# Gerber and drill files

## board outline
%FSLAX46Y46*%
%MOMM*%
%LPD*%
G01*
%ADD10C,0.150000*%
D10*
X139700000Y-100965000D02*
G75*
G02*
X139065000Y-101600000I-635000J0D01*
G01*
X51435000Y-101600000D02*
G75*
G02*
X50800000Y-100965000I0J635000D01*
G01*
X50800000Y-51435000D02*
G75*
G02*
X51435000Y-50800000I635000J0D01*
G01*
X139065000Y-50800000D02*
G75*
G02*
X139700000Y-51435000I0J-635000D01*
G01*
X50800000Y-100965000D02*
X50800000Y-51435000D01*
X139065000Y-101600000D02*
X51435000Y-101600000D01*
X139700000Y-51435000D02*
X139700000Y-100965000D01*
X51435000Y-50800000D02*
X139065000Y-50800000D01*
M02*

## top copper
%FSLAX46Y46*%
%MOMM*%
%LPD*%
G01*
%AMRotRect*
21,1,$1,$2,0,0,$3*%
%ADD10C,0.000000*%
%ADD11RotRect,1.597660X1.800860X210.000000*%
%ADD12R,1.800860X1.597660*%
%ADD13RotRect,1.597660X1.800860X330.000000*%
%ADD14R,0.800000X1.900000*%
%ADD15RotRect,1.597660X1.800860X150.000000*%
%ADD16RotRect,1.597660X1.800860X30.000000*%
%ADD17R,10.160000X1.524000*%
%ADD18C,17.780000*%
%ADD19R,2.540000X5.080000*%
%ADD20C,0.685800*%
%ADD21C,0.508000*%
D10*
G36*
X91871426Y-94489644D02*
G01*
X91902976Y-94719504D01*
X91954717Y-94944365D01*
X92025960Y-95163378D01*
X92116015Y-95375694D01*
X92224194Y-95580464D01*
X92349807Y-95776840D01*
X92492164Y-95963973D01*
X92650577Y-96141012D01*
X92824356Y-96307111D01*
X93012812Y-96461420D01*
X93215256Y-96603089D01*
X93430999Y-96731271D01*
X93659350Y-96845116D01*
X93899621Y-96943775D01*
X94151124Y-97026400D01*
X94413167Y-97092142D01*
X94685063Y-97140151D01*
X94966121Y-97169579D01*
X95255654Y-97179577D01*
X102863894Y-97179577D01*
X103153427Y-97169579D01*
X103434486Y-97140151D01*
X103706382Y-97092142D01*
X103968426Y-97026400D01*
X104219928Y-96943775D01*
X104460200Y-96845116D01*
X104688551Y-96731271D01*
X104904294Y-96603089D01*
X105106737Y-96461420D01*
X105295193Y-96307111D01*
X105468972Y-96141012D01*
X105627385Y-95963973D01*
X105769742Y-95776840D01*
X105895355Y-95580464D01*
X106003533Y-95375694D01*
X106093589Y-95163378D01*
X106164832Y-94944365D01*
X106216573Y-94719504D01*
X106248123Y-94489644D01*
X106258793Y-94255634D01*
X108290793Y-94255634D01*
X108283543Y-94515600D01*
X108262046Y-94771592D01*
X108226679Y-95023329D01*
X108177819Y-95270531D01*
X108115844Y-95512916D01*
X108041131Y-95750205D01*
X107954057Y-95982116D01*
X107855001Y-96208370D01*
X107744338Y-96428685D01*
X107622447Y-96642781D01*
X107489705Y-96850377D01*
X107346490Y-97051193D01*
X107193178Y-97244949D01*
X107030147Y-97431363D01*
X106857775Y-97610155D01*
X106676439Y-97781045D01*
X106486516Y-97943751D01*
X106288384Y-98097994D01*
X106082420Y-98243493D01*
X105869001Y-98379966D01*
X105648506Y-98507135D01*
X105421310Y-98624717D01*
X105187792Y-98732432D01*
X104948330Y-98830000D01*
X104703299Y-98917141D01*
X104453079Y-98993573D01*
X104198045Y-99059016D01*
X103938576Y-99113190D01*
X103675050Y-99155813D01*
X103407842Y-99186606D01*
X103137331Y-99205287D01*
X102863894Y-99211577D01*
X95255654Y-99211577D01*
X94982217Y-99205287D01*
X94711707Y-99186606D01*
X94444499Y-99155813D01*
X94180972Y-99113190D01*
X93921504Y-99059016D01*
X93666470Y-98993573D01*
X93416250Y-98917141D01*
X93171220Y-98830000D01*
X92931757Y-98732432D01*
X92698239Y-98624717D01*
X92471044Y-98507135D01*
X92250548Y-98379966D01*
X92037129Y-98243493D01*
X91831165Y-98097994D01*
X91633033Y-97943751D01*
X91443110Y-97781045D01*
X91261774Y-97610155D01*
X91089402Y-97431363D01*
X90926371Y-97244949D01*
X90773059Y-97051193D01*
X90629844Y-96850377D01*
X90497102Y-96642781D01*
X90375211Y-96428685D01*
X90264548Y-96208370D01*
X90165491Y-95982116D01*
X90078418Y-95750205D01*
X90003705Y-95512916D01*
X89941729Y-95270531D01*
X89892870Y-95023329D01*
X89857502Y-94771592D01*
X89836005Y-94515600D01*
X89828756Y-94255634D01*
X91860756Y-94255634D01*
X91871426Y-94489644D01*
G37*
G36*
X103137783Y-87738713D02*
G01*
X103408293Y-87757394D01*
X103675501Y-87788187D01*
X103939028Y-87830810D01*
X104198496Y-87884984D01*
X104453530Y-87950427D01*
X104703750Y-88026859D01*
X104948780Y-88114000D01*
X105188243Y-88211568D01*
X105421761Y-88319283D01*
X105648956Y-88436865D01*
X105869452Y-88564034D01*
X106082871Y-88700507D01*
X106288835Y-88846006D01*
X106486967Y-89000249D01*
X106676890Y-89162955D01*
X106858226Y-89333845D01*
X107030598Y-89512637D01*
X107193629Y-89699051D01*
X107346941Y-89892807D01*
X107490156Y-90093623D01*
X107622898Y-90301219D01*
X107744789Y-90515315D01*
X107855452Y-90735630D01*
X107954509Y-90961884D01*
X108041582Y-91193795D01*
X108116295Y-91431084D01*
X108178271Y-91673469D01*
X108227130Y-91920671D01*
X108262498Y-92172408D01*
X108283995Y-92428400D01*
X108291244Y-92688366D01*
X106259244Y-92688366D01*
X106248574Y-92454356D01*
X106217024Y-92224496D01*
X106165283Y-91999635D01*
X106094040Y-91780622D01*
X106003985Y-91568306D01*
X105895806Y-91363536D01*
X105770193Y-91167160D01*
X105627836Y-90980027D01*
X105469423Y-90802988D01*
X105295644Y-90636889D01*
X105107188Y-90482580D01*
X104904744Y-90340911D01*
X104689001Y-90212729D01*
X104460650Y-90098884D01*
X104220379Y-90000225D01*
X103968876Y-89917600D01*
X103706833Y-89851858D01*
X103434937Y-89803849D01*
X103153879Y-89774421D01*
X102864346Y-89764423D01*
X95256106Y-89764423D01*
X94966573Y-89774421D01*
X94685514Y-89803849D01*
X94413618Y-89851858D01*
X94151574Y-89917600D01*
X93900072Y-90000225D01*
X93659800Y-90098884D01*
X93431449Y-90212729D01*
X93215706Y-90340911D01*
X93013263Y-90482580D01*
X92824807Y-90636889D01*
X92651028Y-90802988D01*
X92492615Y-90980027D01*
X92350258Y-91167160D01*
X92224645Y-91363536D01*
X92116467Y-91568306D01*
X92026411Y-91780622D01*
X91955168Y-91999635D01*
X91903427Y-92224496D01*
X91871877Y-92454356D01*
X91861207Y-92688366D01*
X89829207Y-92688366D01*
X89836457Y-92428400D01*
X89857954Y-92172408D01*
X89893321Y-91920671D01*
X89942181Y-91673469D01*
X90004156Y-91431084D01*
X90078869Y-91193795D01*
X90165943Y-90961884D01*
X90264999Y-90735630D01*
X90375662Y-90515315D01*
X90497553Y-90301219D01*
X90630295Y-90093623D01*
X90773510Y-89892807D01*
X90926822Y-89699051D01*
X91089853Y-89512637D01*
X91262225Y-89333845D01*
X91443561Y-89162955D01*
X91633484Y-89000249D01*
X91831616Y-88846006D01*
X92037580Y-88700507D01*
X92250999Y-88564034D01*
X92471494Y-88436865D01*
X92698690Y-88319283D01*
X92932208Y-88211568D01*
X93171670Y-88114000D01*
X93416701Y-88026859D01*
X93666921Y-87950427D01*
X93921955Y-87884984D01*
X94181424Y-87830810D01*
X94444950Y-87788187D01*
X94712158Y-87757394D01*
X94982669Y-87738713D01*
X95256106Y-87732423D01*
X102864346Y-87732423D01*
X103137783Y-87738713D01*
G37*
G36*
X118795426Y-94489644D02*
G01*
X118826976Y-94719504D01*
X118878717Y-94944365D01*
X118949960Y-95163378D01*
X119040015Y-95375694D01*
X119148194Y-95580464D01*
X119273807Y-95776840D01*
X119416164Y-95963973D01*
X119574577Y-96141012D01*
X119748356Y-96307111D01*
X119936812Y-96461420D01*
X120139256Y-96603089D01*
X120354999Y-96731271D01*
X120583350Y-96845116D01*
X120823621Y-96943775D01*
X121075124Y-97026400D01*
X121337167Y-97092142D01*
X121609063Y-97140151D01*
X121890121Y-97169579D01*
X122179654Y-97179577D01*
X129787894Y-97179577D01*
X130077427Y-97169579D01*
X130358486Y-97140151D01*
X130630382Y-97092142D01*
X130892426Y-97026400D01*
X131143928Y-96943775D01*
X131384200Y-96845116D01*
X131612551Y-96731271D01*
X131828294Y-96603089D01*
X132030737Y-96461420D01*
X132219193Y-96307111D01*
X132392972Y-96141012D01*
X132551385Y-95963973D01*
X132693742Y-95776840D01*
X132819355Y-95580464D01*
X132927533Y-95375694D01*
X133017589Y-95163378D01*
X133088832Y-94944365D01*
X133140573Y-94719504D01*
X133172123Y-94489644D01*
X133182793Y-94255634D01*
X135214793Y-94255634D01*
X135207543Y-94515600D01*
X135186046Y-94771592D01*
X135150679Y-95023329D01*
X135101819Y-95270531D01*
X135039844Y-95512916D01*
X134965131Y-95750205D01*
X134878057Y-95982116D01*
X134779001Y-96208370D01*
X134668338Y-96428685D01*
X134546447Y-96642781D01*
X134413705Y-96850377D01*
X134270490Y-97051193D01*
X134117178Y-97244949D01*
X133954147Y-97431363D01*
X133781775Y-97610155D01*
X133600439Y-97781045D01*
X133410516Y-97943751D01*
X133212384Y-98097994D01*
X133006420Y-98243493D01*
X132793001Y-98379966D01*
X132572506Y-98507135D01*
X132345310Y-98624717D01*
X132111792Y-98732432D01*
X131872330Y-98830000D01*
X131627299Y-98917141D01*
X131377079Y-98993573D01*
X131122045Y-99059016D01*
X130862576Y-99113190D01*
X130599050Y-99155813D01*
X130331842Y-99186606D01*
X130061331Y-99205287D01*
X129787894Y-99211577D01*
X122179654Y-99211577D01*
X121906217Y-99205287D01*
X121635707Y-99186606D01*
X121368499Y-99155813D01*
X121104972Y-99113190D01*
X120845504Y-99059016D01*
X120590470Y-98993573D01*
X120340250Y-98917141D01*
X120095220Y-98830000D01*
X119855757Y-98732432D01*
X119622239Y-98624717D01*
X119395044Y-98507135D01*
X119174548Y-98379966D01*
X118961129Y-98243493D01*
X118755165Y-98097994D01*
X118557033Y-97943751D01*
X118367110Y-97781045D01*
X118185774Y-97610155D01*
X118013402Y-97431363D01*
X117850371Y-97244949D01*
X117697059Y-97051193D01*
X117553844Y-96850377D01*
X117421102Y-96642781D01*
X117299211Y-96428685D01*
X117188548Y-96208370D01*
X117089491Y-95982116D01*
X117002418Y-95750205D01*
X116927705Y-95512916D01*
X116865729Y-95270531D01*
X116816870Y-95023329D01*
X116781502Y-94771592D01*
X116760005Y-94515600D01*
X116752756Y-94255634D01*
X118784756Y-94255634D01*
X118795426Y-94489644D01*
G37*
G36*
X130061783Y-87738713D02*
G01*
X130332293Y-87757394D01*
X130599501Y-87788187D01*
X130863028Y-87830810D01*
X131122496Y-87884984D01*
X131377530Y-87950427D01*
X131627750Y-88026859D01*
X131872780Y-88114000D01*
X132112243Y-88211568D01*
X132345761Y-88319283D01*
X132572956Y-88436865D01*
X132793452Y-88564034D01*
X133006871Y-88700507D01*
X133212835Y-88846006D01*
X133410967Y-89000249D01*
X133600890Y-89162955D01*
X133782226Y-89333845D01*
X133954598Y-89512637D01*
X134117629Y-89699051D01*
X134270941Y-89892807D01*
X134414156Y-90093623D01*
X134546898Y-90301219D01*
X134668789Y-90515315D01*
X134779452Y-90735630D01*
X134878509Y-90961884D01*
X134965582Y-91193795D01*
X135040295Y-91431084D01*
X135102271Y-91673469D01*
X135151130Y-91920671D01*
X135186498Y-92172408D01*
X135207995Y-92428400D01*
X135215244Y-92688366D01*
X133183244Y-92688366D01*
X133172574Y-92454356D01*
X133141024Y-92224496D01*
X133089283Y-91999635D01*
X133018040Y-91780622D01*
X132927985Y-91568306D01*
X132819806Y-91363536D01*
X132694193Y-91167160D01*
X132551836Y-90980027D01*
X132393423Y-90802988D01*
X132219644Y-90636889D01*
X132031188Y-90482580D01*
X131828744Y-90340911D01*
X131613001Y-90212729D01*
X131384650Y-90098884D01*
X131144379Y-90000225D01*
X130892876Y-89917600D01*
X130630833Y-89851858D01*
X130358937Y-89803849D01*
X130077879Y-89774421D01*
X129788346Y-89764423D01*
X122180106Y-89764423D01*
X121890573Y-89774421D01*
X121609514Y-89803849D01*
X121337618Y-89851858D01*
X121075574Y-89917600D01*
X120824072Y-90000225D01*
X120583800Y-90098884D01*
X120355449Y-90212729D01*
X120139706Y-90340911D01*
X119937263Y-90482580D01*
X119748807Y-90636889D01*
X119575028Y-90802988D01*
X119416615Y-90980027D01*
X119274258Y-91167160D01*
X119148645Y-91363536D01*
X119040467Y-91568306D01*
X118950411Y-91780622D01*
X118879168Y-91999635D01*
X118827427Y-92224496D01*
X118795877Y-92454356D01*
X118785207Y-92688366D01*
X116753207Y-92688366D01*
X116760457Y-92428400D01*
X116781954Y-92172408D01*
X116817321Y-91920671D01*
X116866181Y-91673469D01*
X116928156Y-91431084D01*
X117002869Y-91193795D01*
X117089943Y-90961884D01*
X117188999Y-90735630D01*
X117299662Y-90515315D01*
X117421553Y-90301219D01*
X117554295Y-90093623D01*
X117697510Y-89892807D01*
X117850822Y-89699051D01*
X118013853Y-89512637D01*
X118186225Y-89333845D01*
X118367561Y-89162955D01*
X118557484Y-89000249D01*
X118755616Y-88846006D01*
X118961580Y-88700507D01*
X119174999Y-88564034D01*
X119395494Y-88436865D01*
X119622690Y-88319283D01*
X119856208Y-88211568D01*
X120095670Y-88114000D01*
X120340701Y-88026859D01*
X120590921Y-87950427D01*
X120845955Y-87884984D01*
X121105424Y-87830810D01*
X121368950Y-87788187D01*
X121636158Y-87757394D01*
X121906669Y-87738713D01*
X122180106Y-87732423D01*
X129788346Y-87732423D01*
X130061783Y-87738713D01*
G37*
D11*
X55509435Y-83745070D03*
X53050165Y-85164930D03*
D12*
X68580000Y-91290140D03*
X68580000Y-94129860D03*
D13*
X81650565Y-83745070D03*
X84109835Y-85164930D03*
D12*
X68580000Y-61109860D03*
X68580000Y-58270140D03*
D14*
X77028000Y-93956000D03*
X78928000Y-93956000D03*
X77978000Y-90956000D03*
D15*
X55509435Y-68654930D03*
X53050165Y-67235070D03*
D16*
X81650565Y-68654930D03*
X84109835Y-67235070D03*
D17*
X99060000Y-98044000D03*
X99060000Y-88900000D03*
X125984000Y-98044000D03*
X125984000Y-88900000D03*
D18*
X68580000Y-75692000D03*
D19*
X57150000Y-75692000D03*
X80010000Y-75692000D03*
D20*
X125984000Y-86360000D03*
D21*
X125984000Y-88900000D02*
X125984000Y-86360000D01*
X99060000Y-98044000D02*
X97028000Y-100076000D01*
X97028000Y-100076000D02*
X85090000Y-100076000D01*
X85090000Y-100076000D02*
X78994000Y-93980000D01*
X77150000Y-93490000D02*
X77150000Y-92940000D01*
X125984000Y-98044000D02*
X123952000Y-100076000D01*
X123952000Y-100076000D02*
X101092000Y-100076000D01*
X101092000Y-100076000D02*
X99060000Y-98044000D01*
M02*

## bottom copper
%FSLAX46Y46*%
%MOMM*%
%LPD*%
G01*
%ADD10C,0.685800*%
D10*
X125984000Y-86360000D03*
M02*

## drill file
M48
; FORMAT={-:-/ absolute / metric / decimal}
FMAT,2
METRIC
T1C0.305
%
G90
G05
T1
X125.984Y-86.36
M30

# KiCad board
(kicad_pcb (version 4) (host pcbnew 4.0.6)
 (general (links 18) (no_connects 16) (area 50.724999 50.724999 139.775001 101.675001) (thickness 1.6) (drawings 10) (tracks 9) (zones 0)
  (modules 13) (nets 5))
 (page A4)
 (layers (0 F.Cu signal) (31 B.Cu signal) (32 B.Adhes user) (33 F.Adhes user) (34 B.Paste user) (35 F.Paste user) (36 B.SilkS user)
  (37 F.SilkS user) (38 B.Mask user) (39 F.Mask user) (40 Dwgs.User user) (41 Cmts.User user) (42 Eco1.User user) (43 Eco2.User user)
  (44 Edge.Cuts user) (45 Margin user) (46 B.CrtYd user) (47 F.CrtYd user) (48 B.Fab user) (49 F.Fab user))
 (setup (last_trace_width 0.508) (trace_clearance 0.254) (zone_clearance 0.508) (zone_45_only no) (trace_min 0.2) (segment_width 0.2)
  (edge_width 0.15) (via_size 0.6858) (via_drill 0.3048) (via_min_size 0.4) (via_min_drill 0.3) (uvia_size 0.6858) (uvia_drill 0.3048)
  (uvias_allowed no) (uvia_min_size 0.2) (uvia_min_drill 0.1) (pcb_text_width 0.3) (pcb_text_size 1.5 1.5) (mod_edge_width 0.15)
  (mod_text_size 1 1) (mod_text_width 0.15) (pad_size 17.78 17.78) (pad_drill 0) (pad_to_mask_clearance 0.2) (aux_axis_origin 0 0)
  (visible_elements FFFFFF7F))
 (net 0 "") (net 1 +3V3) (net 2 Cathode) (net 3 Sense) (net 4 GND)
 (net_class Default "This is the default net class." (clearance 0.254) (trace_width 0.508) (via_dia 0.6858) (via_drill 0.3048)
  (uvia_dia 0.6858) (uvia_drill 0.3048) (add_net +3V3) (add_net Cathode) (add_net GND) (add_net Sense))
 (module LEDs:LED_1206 (layer F.Cu) (at 54.2798 84.455 30)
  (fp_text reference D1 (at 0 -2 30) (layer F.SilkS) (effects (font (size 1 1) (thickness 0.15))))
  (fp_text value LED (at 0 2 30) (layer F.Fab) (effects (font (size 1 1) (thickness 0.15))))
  (pad 2 smd rect (at 1.41986 0 210) (size 1.59766 1.80086) (layers F.Cu F.Paste F.Mask) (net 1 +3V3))
  (pad 1 smd rect (at -1.41986 0 210) (size 1.59766 1.80086) (layers F.Cu F.Paste F.Mask) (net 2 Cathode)))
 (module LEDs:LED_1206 (layer F.Cu) (at 68.58 92.71 90)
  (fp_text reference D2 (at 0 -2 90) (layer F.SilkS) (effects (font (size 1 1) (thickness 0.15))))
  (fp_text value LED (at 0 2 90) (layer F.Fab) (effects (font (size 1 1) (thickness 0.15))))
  (pad 2 smd rect (at 1.41986 0 270) (size 1.59766 1.80086) (layers F.Cu F.Paste F.Mask) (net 1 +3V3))
  (pad 1 smd rect (at -1.41986 0 270) (size 1.59766 1.80086) (layers F.Cu F.Paste F.Mask) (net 2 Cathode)))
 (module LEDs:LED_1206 (layer F.Cu) (at 82.8802 84.455 150)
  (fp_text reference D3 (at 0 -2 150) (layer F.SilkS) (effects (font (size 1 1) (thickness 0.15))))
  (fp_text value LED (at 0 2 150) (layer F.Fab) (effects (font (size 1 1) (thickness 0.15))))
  (pad 2 smd rect (at 1.41986 0 330) (size 1.59766 1.80086) (layers F.Cu F.Paste F.Mask) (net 1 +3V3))
  (pad 1 smd rect (at -1.41986 0 330) (size 1.59766 1.80086) (layers F.Cu F.Paste F.Mask) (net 2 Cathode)))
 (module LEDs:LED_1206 (layer F.Cu) (at 68.58 59.69 270)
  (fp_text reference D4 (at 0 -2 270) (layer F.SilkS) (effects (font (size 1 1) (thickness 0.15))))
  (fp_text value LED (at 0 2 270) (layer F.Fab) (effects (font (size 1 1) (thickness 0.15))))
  (pad 2 smd rect (at 1.41986 0 90) (size 1.59766 1.80086) (layers F.Cu F.Paste F.Mask) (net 1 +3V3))
  (pad 1 smd rect (at -1.41986 0 90) (size 1.59766 1.80086) (layers F.Cu F.Paste F.Mask) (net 2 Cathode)))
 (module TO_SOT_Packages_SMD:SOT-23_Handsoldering (layer F.Cu) (at 77.978 92.456 90)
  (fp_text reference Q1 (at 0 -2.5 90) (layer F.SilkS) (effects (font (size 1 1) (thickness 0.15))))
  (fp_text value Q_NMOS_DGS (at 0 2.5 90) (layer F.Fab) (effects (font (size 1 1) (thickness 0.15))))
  (pad 1 smd rect (at -1.5 -0.95 90) (size 1.9 0.8) (layers F.Cu F.Paste F.Mask) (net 2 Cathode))
  (pad 2 smd rect (at -1.5 0.95 90) (size 1.9 0.8) (layers F.Cu F.Paste F.Mask) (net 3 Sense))
  (pad 3 smd rect (at 1.5 0 90) (size 1.9 0.8) (layers F.Cu F.Paste F.Mask) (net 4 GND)))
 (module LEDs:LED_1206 (layer F.Cu) (at 54.2798 67.945 330)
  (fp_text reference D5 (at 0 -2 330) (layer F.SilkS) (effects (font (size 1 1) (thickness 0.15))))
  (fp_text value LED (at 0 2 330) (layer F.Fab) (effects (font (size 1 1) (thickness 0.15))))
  (pad 2 smd rect (at 1.41986 0 150) (size 1.59766 1.80086) (layers F.Cu F.Paste F.Mask) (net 1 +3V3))
  (pad 1 smd rect (at -1.41986 0 150) (size 1.59766 1.80086) (layers F.Cu F.Paste F.Mask) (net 2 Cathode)))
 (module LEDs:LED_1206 (layer F.Cu) (at 82.8802 67.945 210)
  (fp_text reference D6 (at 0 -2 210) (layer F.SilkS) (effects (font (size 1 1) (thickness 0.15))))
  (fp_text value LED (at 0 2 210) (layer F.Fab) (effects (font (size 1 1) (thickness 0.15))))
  (pad 2 smd rect (at 1.41986 0 30) (size 1.59766 1.80086) (layers F.Cu F.Paste F.Mask) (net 1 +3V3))
  (pad 1 smd rect (at -1.41986 0 30) (size 1.59766 1.80086) (layers F.Cu F.Paste F.Mask) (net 2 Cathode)))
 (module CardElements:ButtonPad (layer F.Cu) (at 99.06 96.774 180)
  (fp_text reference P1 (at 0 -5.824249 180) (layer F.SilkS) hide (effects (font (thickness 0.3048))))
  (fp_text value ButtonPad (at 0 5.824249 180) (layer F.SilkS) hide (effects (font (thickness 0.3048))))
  (fp_poly
   (pts (xy -3.803894 -2.437577) (xy -4.077331 -2.431287) (xy -4.347842 -2.412606) (xy -4.61505 -2.381813) (xy -4.878576 -2.33919)
    (xy -5.138045 -2.285016) (xy -5.393079 -2.219573) (xy -5.643299 -2.143141) (xy -5.88833 -2.056) (xy -6.127792 -1.958432)
    (xy -6.36131 -1.850717) (xy -6.588506 -1.733135) (xy -6.809001 -1.605966) (xy -7.02242 -1.469493) (xy -7.228384 -1.323994)
    (xy -7.426516 -1.169751) (xy -7.616439 -1.007045) (xy -7.797775 -0.836155) (xy -7.970147 -0.657363) (xy -8.133178 -0.470949)
    (xy -8.28649 -0.277193) (xy -8.429705 -0.076377) (xy -8.562447 0.131219) (xy -8.684338 0.345315) (xy -8.795001 0.56563)
    (xy -8.894057 0.791884) (xy -8.981131 1.023795) (xy -9.055844 1.261084) (xy -9.117819 1.503469) (xy -9.166679 1.750671)
    (xy -9.202046 2.002408) (xy -9.223543 2.2584) (xy -9.230793 2.518366) (xy -7.198793 2.518366) (xy -7.188123 2.284356)
    (xy -7.156573 2.054496) (xy -7.104832 1.829635) (xy -7.033589 1.610622) (xy -6.943533 1.398306) (xy -6.835355 1.193536)
    (xy -6.709742 0.99716) (xy -6.567385 0.810027) (xy -6.408972 0.632988) (xy -6.235193 0.466889) (xy -6.046737 0.31258)
    (xy -5.844294 0.170911) (xy -5.628551 0.042729) (xy -5.4002 -0.071116) (xy -5.159928 -0.169775) (xy -4.908426 -0.2524)
    (xy -4.646382 -0.318142) (xy -4.374486 -0.366151) (xy -4.093427 -0.395579) (xy -3.803894 -0.405577) (xy 3.804346 -0.405577)
    (xy 4.093879 -0.395579) (xy 4.374937 -0.366151) (xy 4.646833 -0.318142) (xy 4.908876 -0.2524) (xy 5.160379 -0.169775)
    (xy 5.40065 -0.071116) (xy 5.629001 0.042729) (xy 5.844744 0.170911) (xy 6.047188 0.31258) (xy 6.235644 0.466889) (xy 6.409423 0.632988)
    (xy 6.567836 0.810027) (xy 6.710193 0.99716) (xy 6.835806 1.193536) (xy 6.943985 1.398306) (xy 7.03404 1.610622) (xy 7.105283 1.829635)
    (xy 7.157024 2.054496) (xy 7.188574 2.284356) (xy 7.199244 2.518366) (xy 9.231244 2.518366) (xy 9.223995 2.2584) (xy 9.202498 2.002408)
    (xy 9.16713 1.750671) (xy 9.118271 1.503469) (xy 9.056295 1.261084) (xy 8.981582 1.023795) (xy 8.894509 0.791884) (xy 8.795452 0.56563)
    (xy 8.684789 0.345315) (xy 8.562898 0.131219) (xy 8.430156 -0.076377) (xy 8.286941 -0.277193) (xy 8.133629 -0.470949)
    (xy 7.970598 -0.657363) (xy 7.798226 -0.836155) (xy 7.61689 -1.007045) (xy 7.426967 -1.169751) (xy 7.228835 -1.323994)
    (xy 7.022871 -1.469493) (xy 6.809452 -1.605966) (xy 6.588956 -1.733135) (xy 6.361761 -1.850717) (xy 6.128243 -1.958432)
    (xy 5.88878 -2.056) (xy 5.64375 -2.143141) (xy 5.39353 -2.219573) (xy 5.138496 -2.285016) (xy 4.879028 -2.33919) (xy 4.615501 -2.381813)
    (xy 4.348293 -2.412606) (xy 4.077783 -2.431287) (xy 3.804346 -2.437577) (xy -3.803894 -2.437577))
   (layer F.Cu) (width 0))
  (pad 1 smd rect (at 0 -1.27 180) (size 10.16 1.524) (layers F.Cu) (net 3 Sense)))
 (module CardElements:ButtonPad (layer F.Cu) (at 99.06 90.17)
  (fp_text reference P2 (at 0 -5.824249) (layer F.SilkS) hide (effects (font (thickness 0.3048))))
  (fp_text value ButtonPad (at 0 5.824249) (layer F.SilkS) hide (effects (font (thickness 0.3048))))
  (fp_poly
   (pts (xy -3.803894 -2.437577) (xy -4.077331 -2.431287) (xy -4.347842 -2.412606) (xy -4.61505 -2.381813) (xy -4.878576 -2.33919)
    (xy -5.138045 -2.285016) (xy -5.393079 -2.219573) (xy -5.643299 -2.143141) (xy -5.88833 -2.056) (xy -6.127792 -1.958432)
    (xy -6.36131 -1.850717) (xy -6.588506 -1.733135) (xy -6.809001 -1.605966) (xy -7.02242 -1.469493) (xy -7.228384 -1.323994)
    (xy -7.426516 -1.169751) (xy -7.616439 -1.007045) (xy -7.797775 -0.836155) (xy -7.970147 -0.657363) (xy -8.133178 -0.470949)
    (xy -8.28649 -0.277193) (xy -8.429705 -0.076377) (xy -8.562447 0.131219) (xy -8.684338 0.345315) (xy -8.795001 0.56563)
    (xy -8.894057 0.791884) (xy -8.981131 1.023795) (xy -9.055844 1.261084) (xy -9.117819 1.503469) (xy -9.166679 1.750671)
    (xy -9.202046 2.002408) (xy -9.223543 2.2584) (xy -9.230793 2.518366) (xy -7.198793 2.518366) (xy -7.188123 2.284356)
    (xy -7.156573 2.054496) (xy -7.104832 1.829635) (xy -7.033589 1.610622) (xy -6.943533 1.398306) (xy -6.835355 1.193536)
    (xy -6.709742 0.99716) (xy -6.567385 0.810027) (xy -6.408972 0.632988) (xy -6.235193 0.466889) (xy -6.046737 0.31258)
    (xy -5.844294 0.170911) (xy -5.628551 0.042729) (xy -5.4002 -0.071116) (xy -5.159928 -0.169775) (xy -4.908426 -0.2524)
    (xy -4.646382 -0.318142) (xy -4.374486 -0.366151) (xy -4.093427 -0.395579) (xy -3.803894 -0.405577) (xy 3.804346 -0.405577)
    (xy 4.093879 -0.395579) (xy 4.374937 -0.366151) (xy 4.646833 -0.318142) (xy 4.908876 -0.2524) (xy 5.160379 -0.169775)
    (xy 5.40065 -0.071116) (xy 5.629001 0.042729) (xy 5.844744 0.170911) (xy 6.047188 0.31258) (xy 6.235644 0.466889) (xy 6.409423 0.632988)
    (xy 6.567836 0.810027) (xy 6.710193 0.99716) (xy 6.835806 1.193536) (xy 6.943985 1.398306) (xy 7.03404 1.610622) (xy 7.105283 1.829635)
    (xy 7.157024 2.054496) (xy 7.188574 2.284356) (xy 7.199244 2.518366) (xy 9.231244 2.518366) (xy 9.223995 2.2584) (xy 9.202498 2.002408)
    (xy 9.16713 1.750671) (xy 9.118271 1.503469) (xy 9.056295 1.261084) (xy 8.981582 1.023795) (xy 8.894509 0.791884) (xy 8.795452 0.56563)
    (xy 8.684789 0.345315) (xy 8.562898 0.131219) (xy 8.430156 -0.076377) (xy 8.286941 -0.277193) (xy 8.133629 -0.470949)
    (xy 7.970598 -0.657363) (xy 7.798226 -0.836155) (xy 7.61689 -1.007045) (xy 7.426967 -1.169751) (xy 7.228835 -1.323994)
    (xy 7.022871 -1.469493) (xy 6.809452 -1.605966) (xy 6.588956 -1.733135) (xy 6.361761 -1.850717) (xy 6.128243 -1.958432)
    (xy 5.88878 -2.056) (xy 5.64375 -2.143141) (xy 5.39353 -2.219573) (xy 5.138496 -2.285016) (xy 4.879028 -2.33919) (xy 4.615501 -2.381813)
    (xy 4.348293 -2.412606) (xy 4.077783 -2.431287) (xy 3.804346 -2.437577) (xy -3.803894 -2.437577))
   (layer F.Cu) (width 0))
  (pad 1 smd rect (at 0 -1.27) (size 10.16 1.524) (layers F.Cu) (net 4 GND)))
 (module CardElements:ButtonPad (layer F.Cu) (at 125.984 96.774 180)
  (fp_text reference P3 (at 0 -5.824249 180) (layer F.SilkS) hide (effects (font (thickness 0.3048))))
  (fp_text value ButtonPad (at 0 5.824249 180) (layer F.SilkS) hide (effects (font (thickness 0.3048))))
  (fp_poly
   (pts (xy -3.803894 -2.437577) (xy -4.077331 -2.431287) (xy -4.347842 -2.412606) (xy -4.61505 -2.381813) (xy -4.878576 -2.33919)
    (xy -5.138045 -2.285016) (xy -5.393079 -2.219573) (xy -5.643299 -2.143141) (xy -5.88833 -2.056) (xy -6.127792 -1.958432)
    (xy -6.36131 -1.850717) (xy -6.588506 -1.733135) (xy -6.809001 -1.605966) (xy -7.02242 -1.469493) (xy -7.228384 -1.323994)
    (xy -7.426516 -1.169751) (xy -7.616439 -1.007045) (xy -7.797775 -0.836155) (xy -7.970147 -0.657363) (xy -8.133178 -0.470949)
    (xy -8.28649 -0.277193) (xy -8.429705 -0.076377) (xy -8.562447 0.131219) (xy -8.684338 0.345315) (xy -8.795001 0.56563)
    (xy -8.894057 0.791884) (xy -8.981131 1.023795) (xy -9.055844 1.261084) (xy -9.117819 1.503469) (xy -9.166679 1.750671)
    (xy -9.202046 2.002408) (xy -9.223543 2.2584) (xy -9.230793 2.518366) (xy -7.198793 2.518366) (xy -7.188123 2.284356)
    (xy -7.156573 2.054496) (xy -7.104832 1.829635) (xy -7.033589 1.610622) (xy -6.943533 1.398306) (xy -6.835355 1.193536)
    (xy -6.709742 0.99716) (xy -6.567385 0.810027) (xy -6.408972 0.632988) (xy -6.235193 0.466889) (xy -6.046737 0.31258)
    (xy -5.844294 0.170911) (xy -5.628551 0.042729) (xy -5.4002 -0.071116) (xy -5.159928 -0.169775) (xy -4.908426 -0.2524)
    (xy -4.646382 -0.318142) (xy -4.374486 -0.366151) (xy -4.093427 -0.395579) (xy -3.803894 -0.405577) (xy 3.804346 -0.405577)
    (xy 4.093879 -0.395579) (xy 4.374937 -0.366151) (xy 4.646833 -0.318142) (xy 4.908876 -0.2524) (xy 5.160379 -0.169775)
    (xy 5.40065 -0.071116) (xy 5.629001 0.042729) (xy 5.844744 0.170911) (xy 6.047188 0.31258) (xy 6.235644 0.466889) (xy 6.409423 0.632988)
    (xy 6.567836 0.810027) (xy 6.710193 0.99716) (xy 6.835806 1.193536) (xy 6.943985 1.398306) (xy 7.03404 1.610622) (xy 7.105283 1.829635)
    (xy 7.157024 2.054496) (xy 7.188574 2.284356) (xy 7.199244 2.518366) (xy 9.231244 2.518366) (xy 9.223995 2.2584) (xy 9.202498 2.002408)
    (xy 9.16713 1.750671) (xy 9.118271 1.503469) (xy 9.056295 1.261084) (xy 8.981582 1.023795) (xy 8.894509 0.791884) (xy 8.795452 0.56563)
    (xy 8.684789 0.345315) (xy 8.562898 0.131219) (xy 8.430156 -0.076377) (xy 8.286941 -0.277193) (xy 8.133629 -0.470949)
    (xy 7.970598 -0.657363) (xy 7.798226 -0.836155) (xy 7.61689 -1.007045) (xy 7.426967 -1.169751) (xy 7.228835 -1.323994)
    (xy 7.022871 -1.469493) (xy 6.809452 -1.605966) (xy 6.588956 -1.733135) (xy 6.361761 -1.850717) (xy 6.128243 -1.958432)
    (xy 5.88878 -2.056) (xy 5.64375 -2.143141) (xy 5.39353 -2.219573) (xy 5.138496 -2.285016) (xy 4.879028 -2.33919) (xy 4.615501 -2.381813)
    (xy 4.348293 -2.412606) (xy 4.077783 -2.431287) (xy 3.804346 -2.437577) (xy -3.803894 -2.437577))
   (layer F.Cu) (width 0))
  (pad 1 smd rect (at 0 -1.27 180) (size 10.16 1.524) (layers F.Cu) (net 3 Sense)))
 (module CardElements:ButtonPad (layer F.Cu) (at 125.984 90.17)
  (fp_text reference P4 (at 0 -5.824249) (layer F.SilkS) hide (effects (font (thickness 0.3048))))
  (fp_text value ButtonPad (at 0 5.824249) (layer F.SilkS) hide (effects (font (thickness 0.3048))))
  (fp_poly
   (pts (xy -3.803894 -2.437577) (xy -4.077331 -2.431287) (xy -4.347842 -2.412606) (xy -4.61505 -2.381813) (xy -4.878576 -2.33919)
    (xy -5.138045 -2.285016) (xy -5.393079 -2.219573) (xy -5.643299 -2.143141) (xy -5.88833 -2.056) (xy -6.127792 -1.958432)
    (xy -6.36131 -1.850717) (xy -6.588506 -1.733135) (xy -6.809001 -1.605966) (xy -7.02242 -1.469493) (xy -7.228384 -1.323994)
    (xy -7.426516 -1.169751) (xy -7.616439 -1.007045) (xy -7.797775 -0.836155) (xy -7.970147 -0.657363) (xy -8.133178 -0.470949)
    (xy -8.28649 -0.277193) (xy -8.429705 -0.076377) (xy -8.562447 0.131219) (xy -8.684338 0.345315) (xy -8.795001 0.56563)
    (xy -8.894057 0.791884) (xy -8.981131 1.023795) (xy -9.055844 1.261084) (xy -9.117819 1.503469) (xy -9.166679 1.750671)
    (xy -9.202046 2.002408) (xy -9.223543 2.2584) (xy -9.230793 2.518366) (xy -7.198793 2.518366) (xy -7.188123 2.284356)
    (xy -7.156573 2.054496) (xy -7.104832 1.829635) (xy -7.033589 1.610622) (xy -6.943533 1.398306) (xy -6.835355 1.193536)
    (xy -6.709742 0.99716) (xy -6.567385 0.810027) (xy -6.408972 0.632988) (xy -6.235193 0.466889) (xy -6.046737 0.31258)
    (xy -5.844294 0.170911) (xy -5.628551 0.042729) (xy -5.4002 -0.071116) (xy -5.159928 -0.169775) (xy -4.908426 -0.2524)
    (xy -4.646382 -0.318142) (xy -4.374486 -0.366151) (xy -4.093427 -0.395579) (xy -3.803894 -0.405577) (xy 3.804346 -0.405577)
    (xy 4.093879 -0.395579) (xy 4.374937 -0.366151) (xy 4.646833 -0.318142) (xy 4.908876 -0.2524) (xy 5.160379 -0.169775)
    (xy 5.40065 -0.071116) (xy 5.629001 0.042729) (xy 5.844744 0.170911) (xy 6.047188 0.31258) (xy 6.235644 0.466889) (xy 6.409423 0.632988)
    (xy 6.567836 0.810027) (xy 6.710193 0.99716) (xy 6.835806 1.193536) (xy 6.943985 1.398306) (xy 7.03404 1.610622) (xy 7.105283 1.829635)
    (xy 7.157024 2.054496) (xy 7.188574 2.284356) (xy 7.199244 2.518366) (xy 9.231244 2.518366) (xy 9.223995 2.2584) (xy 9.202498 2.002408)
    (xy 9.16713 1.750671) (xy 9.118271 1.503469) (xy 9.056295 1.261084) (xy 8.981582 1.023795) (xy 8.894509 0.791884) (xy 8.795452 0.56563)
    (xy 8.684789 0.345315) (xy 8.562898 0.131219) (xy 8.430156 -0.076377) (xy 8.286941 -0.277193) (xy 8.133629 -0.470949)
    (xy 7.970598 -0.657363) (xy 7.798226 -0.836155) (xy 7.61689 -1.007045) (xy 7.426967 -1.169751) (xy 7.228835 -1.323994)
    (xy 7.022871 -1.469493) (xy 6.809452 -1.605966) (xy 6.588956 -1.733135) (xy 6.361761 -1.850717) (xy 6.128243 -1.958432)
    (xy 5.88878 -2.056) (xy 5.64375 -2.143141) (xy 5.39353 -2.219573) (xy 5.138496 -2.285016) (xy 4.879028 -2.33919) (xy 4.615501 -2.381813)
    (xy 4.348293 -2.412606) (xy 4.077783 -2.431287) (xy 3.804346 -2.437577) (xy -3.803894 -2.437577))
   (layer F.Cu) (width 0))
  (pad 1 smd rect (at 0 -1.27) (size 10.16 1.524) (layers F.Cu) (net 1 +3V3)))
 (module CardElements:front (layer F.Cu) (at 92.71 72.39)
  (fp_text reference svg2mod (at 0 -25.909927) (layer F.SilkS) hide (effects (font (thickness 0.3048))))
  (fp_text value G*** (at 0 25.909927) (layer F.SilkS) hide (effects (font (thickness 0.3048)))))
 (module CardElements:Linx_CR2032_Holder (layer F.Cu) (at 68.58 75.692)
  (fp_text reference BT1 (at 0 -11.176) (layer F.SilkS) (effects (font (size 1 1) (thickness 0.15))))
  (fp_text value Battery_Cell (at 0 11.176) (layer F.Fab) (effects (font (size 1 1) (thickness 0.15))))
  (pad 1 smd circle (at 0 0) (size 17.78 17.78) (layers F.Cu F.Paste F.Mask) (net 1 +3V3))
  (pad 2 smd rect (at -11.43 0) (size 2.54 5.08) (layers F.Cu F.Paste F.Mask) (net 4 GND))
  (pad 2 smd rect (at 11.43 0) (size 2.54 5.08) (layers F.Cu F.Paste F.Mask) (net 4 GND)))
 (gr_arc (start 139.065 100.965) (end 139.7 100.965) (angle 90) (layer Edge.Cuts) (width 0.15))
 (gr_arc (start 51.435 100.965) (end 51.435 101.6) (angle 90) (layer Edge.Cuts) (width 0.15))
 (gr_arc (start 51.435 51.435) (end 50.8 51.435) (angle 90) (layer Edge.Cuts) (width 0.15))
 (gr_arc (start 139.065 51.435) (end 139.065 50.8) (angle 90) (layer Edge.Cuts) (width 0.15))
 (gr_line (start 50.8 100.965) (end 50.8 51.435) (layer Edge.Cuts) (width 0.15))
 (gr_line (start 139.065 101.6) (end 51.435 101.6) (layer Edge.Cuts) (width 0.15))
 (gr_line (start 139.7 51.435) (end 139.7 100.965) (layer Edge.Cuts) (width 0.15))
 (gr_line (start 51.435 50.8) (end 139.065 50.8) (layer Edge.Cuts) (width 0.15))
 (segment (start 125.984 88.9) (end 125.984 86.36) (width 0.508) (layer F.Cu) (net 1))
 (via (at 125.984 86.36) (size 0.6858) (drill 0.3048) (layers F.Cu B.Cu) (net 1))
 (segment (start 99.06 98.044) (end 97.028 100.076) (width 0.508) (layer F.Cu) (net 3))
 (segment (start 97.028 100.076) (end 85.09 100.076) (width 0.508) (layer F.Cu) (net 3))
 (segment (start 85.09 100.076) (end 78.994 93.98) (width 0.508) (layer F.Cu) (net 3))
 (segment (start 77.15 93.49) (end 77.15 92.94) (width 0.508) (layer F.Cu) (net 3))
 (segment (start 125.984 98.044) (end 123.952 100.076) (width 0.508) (layer F.Cu) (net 3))
 (segment (start 123.952 100.076) (end 101.092 100.076) (width 0.508) (layer F.Cu) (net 3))
 (segment (start 101.092 100.076) (end 99.06 98.044) (width 0.508) (layer F.Cu) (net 3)))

